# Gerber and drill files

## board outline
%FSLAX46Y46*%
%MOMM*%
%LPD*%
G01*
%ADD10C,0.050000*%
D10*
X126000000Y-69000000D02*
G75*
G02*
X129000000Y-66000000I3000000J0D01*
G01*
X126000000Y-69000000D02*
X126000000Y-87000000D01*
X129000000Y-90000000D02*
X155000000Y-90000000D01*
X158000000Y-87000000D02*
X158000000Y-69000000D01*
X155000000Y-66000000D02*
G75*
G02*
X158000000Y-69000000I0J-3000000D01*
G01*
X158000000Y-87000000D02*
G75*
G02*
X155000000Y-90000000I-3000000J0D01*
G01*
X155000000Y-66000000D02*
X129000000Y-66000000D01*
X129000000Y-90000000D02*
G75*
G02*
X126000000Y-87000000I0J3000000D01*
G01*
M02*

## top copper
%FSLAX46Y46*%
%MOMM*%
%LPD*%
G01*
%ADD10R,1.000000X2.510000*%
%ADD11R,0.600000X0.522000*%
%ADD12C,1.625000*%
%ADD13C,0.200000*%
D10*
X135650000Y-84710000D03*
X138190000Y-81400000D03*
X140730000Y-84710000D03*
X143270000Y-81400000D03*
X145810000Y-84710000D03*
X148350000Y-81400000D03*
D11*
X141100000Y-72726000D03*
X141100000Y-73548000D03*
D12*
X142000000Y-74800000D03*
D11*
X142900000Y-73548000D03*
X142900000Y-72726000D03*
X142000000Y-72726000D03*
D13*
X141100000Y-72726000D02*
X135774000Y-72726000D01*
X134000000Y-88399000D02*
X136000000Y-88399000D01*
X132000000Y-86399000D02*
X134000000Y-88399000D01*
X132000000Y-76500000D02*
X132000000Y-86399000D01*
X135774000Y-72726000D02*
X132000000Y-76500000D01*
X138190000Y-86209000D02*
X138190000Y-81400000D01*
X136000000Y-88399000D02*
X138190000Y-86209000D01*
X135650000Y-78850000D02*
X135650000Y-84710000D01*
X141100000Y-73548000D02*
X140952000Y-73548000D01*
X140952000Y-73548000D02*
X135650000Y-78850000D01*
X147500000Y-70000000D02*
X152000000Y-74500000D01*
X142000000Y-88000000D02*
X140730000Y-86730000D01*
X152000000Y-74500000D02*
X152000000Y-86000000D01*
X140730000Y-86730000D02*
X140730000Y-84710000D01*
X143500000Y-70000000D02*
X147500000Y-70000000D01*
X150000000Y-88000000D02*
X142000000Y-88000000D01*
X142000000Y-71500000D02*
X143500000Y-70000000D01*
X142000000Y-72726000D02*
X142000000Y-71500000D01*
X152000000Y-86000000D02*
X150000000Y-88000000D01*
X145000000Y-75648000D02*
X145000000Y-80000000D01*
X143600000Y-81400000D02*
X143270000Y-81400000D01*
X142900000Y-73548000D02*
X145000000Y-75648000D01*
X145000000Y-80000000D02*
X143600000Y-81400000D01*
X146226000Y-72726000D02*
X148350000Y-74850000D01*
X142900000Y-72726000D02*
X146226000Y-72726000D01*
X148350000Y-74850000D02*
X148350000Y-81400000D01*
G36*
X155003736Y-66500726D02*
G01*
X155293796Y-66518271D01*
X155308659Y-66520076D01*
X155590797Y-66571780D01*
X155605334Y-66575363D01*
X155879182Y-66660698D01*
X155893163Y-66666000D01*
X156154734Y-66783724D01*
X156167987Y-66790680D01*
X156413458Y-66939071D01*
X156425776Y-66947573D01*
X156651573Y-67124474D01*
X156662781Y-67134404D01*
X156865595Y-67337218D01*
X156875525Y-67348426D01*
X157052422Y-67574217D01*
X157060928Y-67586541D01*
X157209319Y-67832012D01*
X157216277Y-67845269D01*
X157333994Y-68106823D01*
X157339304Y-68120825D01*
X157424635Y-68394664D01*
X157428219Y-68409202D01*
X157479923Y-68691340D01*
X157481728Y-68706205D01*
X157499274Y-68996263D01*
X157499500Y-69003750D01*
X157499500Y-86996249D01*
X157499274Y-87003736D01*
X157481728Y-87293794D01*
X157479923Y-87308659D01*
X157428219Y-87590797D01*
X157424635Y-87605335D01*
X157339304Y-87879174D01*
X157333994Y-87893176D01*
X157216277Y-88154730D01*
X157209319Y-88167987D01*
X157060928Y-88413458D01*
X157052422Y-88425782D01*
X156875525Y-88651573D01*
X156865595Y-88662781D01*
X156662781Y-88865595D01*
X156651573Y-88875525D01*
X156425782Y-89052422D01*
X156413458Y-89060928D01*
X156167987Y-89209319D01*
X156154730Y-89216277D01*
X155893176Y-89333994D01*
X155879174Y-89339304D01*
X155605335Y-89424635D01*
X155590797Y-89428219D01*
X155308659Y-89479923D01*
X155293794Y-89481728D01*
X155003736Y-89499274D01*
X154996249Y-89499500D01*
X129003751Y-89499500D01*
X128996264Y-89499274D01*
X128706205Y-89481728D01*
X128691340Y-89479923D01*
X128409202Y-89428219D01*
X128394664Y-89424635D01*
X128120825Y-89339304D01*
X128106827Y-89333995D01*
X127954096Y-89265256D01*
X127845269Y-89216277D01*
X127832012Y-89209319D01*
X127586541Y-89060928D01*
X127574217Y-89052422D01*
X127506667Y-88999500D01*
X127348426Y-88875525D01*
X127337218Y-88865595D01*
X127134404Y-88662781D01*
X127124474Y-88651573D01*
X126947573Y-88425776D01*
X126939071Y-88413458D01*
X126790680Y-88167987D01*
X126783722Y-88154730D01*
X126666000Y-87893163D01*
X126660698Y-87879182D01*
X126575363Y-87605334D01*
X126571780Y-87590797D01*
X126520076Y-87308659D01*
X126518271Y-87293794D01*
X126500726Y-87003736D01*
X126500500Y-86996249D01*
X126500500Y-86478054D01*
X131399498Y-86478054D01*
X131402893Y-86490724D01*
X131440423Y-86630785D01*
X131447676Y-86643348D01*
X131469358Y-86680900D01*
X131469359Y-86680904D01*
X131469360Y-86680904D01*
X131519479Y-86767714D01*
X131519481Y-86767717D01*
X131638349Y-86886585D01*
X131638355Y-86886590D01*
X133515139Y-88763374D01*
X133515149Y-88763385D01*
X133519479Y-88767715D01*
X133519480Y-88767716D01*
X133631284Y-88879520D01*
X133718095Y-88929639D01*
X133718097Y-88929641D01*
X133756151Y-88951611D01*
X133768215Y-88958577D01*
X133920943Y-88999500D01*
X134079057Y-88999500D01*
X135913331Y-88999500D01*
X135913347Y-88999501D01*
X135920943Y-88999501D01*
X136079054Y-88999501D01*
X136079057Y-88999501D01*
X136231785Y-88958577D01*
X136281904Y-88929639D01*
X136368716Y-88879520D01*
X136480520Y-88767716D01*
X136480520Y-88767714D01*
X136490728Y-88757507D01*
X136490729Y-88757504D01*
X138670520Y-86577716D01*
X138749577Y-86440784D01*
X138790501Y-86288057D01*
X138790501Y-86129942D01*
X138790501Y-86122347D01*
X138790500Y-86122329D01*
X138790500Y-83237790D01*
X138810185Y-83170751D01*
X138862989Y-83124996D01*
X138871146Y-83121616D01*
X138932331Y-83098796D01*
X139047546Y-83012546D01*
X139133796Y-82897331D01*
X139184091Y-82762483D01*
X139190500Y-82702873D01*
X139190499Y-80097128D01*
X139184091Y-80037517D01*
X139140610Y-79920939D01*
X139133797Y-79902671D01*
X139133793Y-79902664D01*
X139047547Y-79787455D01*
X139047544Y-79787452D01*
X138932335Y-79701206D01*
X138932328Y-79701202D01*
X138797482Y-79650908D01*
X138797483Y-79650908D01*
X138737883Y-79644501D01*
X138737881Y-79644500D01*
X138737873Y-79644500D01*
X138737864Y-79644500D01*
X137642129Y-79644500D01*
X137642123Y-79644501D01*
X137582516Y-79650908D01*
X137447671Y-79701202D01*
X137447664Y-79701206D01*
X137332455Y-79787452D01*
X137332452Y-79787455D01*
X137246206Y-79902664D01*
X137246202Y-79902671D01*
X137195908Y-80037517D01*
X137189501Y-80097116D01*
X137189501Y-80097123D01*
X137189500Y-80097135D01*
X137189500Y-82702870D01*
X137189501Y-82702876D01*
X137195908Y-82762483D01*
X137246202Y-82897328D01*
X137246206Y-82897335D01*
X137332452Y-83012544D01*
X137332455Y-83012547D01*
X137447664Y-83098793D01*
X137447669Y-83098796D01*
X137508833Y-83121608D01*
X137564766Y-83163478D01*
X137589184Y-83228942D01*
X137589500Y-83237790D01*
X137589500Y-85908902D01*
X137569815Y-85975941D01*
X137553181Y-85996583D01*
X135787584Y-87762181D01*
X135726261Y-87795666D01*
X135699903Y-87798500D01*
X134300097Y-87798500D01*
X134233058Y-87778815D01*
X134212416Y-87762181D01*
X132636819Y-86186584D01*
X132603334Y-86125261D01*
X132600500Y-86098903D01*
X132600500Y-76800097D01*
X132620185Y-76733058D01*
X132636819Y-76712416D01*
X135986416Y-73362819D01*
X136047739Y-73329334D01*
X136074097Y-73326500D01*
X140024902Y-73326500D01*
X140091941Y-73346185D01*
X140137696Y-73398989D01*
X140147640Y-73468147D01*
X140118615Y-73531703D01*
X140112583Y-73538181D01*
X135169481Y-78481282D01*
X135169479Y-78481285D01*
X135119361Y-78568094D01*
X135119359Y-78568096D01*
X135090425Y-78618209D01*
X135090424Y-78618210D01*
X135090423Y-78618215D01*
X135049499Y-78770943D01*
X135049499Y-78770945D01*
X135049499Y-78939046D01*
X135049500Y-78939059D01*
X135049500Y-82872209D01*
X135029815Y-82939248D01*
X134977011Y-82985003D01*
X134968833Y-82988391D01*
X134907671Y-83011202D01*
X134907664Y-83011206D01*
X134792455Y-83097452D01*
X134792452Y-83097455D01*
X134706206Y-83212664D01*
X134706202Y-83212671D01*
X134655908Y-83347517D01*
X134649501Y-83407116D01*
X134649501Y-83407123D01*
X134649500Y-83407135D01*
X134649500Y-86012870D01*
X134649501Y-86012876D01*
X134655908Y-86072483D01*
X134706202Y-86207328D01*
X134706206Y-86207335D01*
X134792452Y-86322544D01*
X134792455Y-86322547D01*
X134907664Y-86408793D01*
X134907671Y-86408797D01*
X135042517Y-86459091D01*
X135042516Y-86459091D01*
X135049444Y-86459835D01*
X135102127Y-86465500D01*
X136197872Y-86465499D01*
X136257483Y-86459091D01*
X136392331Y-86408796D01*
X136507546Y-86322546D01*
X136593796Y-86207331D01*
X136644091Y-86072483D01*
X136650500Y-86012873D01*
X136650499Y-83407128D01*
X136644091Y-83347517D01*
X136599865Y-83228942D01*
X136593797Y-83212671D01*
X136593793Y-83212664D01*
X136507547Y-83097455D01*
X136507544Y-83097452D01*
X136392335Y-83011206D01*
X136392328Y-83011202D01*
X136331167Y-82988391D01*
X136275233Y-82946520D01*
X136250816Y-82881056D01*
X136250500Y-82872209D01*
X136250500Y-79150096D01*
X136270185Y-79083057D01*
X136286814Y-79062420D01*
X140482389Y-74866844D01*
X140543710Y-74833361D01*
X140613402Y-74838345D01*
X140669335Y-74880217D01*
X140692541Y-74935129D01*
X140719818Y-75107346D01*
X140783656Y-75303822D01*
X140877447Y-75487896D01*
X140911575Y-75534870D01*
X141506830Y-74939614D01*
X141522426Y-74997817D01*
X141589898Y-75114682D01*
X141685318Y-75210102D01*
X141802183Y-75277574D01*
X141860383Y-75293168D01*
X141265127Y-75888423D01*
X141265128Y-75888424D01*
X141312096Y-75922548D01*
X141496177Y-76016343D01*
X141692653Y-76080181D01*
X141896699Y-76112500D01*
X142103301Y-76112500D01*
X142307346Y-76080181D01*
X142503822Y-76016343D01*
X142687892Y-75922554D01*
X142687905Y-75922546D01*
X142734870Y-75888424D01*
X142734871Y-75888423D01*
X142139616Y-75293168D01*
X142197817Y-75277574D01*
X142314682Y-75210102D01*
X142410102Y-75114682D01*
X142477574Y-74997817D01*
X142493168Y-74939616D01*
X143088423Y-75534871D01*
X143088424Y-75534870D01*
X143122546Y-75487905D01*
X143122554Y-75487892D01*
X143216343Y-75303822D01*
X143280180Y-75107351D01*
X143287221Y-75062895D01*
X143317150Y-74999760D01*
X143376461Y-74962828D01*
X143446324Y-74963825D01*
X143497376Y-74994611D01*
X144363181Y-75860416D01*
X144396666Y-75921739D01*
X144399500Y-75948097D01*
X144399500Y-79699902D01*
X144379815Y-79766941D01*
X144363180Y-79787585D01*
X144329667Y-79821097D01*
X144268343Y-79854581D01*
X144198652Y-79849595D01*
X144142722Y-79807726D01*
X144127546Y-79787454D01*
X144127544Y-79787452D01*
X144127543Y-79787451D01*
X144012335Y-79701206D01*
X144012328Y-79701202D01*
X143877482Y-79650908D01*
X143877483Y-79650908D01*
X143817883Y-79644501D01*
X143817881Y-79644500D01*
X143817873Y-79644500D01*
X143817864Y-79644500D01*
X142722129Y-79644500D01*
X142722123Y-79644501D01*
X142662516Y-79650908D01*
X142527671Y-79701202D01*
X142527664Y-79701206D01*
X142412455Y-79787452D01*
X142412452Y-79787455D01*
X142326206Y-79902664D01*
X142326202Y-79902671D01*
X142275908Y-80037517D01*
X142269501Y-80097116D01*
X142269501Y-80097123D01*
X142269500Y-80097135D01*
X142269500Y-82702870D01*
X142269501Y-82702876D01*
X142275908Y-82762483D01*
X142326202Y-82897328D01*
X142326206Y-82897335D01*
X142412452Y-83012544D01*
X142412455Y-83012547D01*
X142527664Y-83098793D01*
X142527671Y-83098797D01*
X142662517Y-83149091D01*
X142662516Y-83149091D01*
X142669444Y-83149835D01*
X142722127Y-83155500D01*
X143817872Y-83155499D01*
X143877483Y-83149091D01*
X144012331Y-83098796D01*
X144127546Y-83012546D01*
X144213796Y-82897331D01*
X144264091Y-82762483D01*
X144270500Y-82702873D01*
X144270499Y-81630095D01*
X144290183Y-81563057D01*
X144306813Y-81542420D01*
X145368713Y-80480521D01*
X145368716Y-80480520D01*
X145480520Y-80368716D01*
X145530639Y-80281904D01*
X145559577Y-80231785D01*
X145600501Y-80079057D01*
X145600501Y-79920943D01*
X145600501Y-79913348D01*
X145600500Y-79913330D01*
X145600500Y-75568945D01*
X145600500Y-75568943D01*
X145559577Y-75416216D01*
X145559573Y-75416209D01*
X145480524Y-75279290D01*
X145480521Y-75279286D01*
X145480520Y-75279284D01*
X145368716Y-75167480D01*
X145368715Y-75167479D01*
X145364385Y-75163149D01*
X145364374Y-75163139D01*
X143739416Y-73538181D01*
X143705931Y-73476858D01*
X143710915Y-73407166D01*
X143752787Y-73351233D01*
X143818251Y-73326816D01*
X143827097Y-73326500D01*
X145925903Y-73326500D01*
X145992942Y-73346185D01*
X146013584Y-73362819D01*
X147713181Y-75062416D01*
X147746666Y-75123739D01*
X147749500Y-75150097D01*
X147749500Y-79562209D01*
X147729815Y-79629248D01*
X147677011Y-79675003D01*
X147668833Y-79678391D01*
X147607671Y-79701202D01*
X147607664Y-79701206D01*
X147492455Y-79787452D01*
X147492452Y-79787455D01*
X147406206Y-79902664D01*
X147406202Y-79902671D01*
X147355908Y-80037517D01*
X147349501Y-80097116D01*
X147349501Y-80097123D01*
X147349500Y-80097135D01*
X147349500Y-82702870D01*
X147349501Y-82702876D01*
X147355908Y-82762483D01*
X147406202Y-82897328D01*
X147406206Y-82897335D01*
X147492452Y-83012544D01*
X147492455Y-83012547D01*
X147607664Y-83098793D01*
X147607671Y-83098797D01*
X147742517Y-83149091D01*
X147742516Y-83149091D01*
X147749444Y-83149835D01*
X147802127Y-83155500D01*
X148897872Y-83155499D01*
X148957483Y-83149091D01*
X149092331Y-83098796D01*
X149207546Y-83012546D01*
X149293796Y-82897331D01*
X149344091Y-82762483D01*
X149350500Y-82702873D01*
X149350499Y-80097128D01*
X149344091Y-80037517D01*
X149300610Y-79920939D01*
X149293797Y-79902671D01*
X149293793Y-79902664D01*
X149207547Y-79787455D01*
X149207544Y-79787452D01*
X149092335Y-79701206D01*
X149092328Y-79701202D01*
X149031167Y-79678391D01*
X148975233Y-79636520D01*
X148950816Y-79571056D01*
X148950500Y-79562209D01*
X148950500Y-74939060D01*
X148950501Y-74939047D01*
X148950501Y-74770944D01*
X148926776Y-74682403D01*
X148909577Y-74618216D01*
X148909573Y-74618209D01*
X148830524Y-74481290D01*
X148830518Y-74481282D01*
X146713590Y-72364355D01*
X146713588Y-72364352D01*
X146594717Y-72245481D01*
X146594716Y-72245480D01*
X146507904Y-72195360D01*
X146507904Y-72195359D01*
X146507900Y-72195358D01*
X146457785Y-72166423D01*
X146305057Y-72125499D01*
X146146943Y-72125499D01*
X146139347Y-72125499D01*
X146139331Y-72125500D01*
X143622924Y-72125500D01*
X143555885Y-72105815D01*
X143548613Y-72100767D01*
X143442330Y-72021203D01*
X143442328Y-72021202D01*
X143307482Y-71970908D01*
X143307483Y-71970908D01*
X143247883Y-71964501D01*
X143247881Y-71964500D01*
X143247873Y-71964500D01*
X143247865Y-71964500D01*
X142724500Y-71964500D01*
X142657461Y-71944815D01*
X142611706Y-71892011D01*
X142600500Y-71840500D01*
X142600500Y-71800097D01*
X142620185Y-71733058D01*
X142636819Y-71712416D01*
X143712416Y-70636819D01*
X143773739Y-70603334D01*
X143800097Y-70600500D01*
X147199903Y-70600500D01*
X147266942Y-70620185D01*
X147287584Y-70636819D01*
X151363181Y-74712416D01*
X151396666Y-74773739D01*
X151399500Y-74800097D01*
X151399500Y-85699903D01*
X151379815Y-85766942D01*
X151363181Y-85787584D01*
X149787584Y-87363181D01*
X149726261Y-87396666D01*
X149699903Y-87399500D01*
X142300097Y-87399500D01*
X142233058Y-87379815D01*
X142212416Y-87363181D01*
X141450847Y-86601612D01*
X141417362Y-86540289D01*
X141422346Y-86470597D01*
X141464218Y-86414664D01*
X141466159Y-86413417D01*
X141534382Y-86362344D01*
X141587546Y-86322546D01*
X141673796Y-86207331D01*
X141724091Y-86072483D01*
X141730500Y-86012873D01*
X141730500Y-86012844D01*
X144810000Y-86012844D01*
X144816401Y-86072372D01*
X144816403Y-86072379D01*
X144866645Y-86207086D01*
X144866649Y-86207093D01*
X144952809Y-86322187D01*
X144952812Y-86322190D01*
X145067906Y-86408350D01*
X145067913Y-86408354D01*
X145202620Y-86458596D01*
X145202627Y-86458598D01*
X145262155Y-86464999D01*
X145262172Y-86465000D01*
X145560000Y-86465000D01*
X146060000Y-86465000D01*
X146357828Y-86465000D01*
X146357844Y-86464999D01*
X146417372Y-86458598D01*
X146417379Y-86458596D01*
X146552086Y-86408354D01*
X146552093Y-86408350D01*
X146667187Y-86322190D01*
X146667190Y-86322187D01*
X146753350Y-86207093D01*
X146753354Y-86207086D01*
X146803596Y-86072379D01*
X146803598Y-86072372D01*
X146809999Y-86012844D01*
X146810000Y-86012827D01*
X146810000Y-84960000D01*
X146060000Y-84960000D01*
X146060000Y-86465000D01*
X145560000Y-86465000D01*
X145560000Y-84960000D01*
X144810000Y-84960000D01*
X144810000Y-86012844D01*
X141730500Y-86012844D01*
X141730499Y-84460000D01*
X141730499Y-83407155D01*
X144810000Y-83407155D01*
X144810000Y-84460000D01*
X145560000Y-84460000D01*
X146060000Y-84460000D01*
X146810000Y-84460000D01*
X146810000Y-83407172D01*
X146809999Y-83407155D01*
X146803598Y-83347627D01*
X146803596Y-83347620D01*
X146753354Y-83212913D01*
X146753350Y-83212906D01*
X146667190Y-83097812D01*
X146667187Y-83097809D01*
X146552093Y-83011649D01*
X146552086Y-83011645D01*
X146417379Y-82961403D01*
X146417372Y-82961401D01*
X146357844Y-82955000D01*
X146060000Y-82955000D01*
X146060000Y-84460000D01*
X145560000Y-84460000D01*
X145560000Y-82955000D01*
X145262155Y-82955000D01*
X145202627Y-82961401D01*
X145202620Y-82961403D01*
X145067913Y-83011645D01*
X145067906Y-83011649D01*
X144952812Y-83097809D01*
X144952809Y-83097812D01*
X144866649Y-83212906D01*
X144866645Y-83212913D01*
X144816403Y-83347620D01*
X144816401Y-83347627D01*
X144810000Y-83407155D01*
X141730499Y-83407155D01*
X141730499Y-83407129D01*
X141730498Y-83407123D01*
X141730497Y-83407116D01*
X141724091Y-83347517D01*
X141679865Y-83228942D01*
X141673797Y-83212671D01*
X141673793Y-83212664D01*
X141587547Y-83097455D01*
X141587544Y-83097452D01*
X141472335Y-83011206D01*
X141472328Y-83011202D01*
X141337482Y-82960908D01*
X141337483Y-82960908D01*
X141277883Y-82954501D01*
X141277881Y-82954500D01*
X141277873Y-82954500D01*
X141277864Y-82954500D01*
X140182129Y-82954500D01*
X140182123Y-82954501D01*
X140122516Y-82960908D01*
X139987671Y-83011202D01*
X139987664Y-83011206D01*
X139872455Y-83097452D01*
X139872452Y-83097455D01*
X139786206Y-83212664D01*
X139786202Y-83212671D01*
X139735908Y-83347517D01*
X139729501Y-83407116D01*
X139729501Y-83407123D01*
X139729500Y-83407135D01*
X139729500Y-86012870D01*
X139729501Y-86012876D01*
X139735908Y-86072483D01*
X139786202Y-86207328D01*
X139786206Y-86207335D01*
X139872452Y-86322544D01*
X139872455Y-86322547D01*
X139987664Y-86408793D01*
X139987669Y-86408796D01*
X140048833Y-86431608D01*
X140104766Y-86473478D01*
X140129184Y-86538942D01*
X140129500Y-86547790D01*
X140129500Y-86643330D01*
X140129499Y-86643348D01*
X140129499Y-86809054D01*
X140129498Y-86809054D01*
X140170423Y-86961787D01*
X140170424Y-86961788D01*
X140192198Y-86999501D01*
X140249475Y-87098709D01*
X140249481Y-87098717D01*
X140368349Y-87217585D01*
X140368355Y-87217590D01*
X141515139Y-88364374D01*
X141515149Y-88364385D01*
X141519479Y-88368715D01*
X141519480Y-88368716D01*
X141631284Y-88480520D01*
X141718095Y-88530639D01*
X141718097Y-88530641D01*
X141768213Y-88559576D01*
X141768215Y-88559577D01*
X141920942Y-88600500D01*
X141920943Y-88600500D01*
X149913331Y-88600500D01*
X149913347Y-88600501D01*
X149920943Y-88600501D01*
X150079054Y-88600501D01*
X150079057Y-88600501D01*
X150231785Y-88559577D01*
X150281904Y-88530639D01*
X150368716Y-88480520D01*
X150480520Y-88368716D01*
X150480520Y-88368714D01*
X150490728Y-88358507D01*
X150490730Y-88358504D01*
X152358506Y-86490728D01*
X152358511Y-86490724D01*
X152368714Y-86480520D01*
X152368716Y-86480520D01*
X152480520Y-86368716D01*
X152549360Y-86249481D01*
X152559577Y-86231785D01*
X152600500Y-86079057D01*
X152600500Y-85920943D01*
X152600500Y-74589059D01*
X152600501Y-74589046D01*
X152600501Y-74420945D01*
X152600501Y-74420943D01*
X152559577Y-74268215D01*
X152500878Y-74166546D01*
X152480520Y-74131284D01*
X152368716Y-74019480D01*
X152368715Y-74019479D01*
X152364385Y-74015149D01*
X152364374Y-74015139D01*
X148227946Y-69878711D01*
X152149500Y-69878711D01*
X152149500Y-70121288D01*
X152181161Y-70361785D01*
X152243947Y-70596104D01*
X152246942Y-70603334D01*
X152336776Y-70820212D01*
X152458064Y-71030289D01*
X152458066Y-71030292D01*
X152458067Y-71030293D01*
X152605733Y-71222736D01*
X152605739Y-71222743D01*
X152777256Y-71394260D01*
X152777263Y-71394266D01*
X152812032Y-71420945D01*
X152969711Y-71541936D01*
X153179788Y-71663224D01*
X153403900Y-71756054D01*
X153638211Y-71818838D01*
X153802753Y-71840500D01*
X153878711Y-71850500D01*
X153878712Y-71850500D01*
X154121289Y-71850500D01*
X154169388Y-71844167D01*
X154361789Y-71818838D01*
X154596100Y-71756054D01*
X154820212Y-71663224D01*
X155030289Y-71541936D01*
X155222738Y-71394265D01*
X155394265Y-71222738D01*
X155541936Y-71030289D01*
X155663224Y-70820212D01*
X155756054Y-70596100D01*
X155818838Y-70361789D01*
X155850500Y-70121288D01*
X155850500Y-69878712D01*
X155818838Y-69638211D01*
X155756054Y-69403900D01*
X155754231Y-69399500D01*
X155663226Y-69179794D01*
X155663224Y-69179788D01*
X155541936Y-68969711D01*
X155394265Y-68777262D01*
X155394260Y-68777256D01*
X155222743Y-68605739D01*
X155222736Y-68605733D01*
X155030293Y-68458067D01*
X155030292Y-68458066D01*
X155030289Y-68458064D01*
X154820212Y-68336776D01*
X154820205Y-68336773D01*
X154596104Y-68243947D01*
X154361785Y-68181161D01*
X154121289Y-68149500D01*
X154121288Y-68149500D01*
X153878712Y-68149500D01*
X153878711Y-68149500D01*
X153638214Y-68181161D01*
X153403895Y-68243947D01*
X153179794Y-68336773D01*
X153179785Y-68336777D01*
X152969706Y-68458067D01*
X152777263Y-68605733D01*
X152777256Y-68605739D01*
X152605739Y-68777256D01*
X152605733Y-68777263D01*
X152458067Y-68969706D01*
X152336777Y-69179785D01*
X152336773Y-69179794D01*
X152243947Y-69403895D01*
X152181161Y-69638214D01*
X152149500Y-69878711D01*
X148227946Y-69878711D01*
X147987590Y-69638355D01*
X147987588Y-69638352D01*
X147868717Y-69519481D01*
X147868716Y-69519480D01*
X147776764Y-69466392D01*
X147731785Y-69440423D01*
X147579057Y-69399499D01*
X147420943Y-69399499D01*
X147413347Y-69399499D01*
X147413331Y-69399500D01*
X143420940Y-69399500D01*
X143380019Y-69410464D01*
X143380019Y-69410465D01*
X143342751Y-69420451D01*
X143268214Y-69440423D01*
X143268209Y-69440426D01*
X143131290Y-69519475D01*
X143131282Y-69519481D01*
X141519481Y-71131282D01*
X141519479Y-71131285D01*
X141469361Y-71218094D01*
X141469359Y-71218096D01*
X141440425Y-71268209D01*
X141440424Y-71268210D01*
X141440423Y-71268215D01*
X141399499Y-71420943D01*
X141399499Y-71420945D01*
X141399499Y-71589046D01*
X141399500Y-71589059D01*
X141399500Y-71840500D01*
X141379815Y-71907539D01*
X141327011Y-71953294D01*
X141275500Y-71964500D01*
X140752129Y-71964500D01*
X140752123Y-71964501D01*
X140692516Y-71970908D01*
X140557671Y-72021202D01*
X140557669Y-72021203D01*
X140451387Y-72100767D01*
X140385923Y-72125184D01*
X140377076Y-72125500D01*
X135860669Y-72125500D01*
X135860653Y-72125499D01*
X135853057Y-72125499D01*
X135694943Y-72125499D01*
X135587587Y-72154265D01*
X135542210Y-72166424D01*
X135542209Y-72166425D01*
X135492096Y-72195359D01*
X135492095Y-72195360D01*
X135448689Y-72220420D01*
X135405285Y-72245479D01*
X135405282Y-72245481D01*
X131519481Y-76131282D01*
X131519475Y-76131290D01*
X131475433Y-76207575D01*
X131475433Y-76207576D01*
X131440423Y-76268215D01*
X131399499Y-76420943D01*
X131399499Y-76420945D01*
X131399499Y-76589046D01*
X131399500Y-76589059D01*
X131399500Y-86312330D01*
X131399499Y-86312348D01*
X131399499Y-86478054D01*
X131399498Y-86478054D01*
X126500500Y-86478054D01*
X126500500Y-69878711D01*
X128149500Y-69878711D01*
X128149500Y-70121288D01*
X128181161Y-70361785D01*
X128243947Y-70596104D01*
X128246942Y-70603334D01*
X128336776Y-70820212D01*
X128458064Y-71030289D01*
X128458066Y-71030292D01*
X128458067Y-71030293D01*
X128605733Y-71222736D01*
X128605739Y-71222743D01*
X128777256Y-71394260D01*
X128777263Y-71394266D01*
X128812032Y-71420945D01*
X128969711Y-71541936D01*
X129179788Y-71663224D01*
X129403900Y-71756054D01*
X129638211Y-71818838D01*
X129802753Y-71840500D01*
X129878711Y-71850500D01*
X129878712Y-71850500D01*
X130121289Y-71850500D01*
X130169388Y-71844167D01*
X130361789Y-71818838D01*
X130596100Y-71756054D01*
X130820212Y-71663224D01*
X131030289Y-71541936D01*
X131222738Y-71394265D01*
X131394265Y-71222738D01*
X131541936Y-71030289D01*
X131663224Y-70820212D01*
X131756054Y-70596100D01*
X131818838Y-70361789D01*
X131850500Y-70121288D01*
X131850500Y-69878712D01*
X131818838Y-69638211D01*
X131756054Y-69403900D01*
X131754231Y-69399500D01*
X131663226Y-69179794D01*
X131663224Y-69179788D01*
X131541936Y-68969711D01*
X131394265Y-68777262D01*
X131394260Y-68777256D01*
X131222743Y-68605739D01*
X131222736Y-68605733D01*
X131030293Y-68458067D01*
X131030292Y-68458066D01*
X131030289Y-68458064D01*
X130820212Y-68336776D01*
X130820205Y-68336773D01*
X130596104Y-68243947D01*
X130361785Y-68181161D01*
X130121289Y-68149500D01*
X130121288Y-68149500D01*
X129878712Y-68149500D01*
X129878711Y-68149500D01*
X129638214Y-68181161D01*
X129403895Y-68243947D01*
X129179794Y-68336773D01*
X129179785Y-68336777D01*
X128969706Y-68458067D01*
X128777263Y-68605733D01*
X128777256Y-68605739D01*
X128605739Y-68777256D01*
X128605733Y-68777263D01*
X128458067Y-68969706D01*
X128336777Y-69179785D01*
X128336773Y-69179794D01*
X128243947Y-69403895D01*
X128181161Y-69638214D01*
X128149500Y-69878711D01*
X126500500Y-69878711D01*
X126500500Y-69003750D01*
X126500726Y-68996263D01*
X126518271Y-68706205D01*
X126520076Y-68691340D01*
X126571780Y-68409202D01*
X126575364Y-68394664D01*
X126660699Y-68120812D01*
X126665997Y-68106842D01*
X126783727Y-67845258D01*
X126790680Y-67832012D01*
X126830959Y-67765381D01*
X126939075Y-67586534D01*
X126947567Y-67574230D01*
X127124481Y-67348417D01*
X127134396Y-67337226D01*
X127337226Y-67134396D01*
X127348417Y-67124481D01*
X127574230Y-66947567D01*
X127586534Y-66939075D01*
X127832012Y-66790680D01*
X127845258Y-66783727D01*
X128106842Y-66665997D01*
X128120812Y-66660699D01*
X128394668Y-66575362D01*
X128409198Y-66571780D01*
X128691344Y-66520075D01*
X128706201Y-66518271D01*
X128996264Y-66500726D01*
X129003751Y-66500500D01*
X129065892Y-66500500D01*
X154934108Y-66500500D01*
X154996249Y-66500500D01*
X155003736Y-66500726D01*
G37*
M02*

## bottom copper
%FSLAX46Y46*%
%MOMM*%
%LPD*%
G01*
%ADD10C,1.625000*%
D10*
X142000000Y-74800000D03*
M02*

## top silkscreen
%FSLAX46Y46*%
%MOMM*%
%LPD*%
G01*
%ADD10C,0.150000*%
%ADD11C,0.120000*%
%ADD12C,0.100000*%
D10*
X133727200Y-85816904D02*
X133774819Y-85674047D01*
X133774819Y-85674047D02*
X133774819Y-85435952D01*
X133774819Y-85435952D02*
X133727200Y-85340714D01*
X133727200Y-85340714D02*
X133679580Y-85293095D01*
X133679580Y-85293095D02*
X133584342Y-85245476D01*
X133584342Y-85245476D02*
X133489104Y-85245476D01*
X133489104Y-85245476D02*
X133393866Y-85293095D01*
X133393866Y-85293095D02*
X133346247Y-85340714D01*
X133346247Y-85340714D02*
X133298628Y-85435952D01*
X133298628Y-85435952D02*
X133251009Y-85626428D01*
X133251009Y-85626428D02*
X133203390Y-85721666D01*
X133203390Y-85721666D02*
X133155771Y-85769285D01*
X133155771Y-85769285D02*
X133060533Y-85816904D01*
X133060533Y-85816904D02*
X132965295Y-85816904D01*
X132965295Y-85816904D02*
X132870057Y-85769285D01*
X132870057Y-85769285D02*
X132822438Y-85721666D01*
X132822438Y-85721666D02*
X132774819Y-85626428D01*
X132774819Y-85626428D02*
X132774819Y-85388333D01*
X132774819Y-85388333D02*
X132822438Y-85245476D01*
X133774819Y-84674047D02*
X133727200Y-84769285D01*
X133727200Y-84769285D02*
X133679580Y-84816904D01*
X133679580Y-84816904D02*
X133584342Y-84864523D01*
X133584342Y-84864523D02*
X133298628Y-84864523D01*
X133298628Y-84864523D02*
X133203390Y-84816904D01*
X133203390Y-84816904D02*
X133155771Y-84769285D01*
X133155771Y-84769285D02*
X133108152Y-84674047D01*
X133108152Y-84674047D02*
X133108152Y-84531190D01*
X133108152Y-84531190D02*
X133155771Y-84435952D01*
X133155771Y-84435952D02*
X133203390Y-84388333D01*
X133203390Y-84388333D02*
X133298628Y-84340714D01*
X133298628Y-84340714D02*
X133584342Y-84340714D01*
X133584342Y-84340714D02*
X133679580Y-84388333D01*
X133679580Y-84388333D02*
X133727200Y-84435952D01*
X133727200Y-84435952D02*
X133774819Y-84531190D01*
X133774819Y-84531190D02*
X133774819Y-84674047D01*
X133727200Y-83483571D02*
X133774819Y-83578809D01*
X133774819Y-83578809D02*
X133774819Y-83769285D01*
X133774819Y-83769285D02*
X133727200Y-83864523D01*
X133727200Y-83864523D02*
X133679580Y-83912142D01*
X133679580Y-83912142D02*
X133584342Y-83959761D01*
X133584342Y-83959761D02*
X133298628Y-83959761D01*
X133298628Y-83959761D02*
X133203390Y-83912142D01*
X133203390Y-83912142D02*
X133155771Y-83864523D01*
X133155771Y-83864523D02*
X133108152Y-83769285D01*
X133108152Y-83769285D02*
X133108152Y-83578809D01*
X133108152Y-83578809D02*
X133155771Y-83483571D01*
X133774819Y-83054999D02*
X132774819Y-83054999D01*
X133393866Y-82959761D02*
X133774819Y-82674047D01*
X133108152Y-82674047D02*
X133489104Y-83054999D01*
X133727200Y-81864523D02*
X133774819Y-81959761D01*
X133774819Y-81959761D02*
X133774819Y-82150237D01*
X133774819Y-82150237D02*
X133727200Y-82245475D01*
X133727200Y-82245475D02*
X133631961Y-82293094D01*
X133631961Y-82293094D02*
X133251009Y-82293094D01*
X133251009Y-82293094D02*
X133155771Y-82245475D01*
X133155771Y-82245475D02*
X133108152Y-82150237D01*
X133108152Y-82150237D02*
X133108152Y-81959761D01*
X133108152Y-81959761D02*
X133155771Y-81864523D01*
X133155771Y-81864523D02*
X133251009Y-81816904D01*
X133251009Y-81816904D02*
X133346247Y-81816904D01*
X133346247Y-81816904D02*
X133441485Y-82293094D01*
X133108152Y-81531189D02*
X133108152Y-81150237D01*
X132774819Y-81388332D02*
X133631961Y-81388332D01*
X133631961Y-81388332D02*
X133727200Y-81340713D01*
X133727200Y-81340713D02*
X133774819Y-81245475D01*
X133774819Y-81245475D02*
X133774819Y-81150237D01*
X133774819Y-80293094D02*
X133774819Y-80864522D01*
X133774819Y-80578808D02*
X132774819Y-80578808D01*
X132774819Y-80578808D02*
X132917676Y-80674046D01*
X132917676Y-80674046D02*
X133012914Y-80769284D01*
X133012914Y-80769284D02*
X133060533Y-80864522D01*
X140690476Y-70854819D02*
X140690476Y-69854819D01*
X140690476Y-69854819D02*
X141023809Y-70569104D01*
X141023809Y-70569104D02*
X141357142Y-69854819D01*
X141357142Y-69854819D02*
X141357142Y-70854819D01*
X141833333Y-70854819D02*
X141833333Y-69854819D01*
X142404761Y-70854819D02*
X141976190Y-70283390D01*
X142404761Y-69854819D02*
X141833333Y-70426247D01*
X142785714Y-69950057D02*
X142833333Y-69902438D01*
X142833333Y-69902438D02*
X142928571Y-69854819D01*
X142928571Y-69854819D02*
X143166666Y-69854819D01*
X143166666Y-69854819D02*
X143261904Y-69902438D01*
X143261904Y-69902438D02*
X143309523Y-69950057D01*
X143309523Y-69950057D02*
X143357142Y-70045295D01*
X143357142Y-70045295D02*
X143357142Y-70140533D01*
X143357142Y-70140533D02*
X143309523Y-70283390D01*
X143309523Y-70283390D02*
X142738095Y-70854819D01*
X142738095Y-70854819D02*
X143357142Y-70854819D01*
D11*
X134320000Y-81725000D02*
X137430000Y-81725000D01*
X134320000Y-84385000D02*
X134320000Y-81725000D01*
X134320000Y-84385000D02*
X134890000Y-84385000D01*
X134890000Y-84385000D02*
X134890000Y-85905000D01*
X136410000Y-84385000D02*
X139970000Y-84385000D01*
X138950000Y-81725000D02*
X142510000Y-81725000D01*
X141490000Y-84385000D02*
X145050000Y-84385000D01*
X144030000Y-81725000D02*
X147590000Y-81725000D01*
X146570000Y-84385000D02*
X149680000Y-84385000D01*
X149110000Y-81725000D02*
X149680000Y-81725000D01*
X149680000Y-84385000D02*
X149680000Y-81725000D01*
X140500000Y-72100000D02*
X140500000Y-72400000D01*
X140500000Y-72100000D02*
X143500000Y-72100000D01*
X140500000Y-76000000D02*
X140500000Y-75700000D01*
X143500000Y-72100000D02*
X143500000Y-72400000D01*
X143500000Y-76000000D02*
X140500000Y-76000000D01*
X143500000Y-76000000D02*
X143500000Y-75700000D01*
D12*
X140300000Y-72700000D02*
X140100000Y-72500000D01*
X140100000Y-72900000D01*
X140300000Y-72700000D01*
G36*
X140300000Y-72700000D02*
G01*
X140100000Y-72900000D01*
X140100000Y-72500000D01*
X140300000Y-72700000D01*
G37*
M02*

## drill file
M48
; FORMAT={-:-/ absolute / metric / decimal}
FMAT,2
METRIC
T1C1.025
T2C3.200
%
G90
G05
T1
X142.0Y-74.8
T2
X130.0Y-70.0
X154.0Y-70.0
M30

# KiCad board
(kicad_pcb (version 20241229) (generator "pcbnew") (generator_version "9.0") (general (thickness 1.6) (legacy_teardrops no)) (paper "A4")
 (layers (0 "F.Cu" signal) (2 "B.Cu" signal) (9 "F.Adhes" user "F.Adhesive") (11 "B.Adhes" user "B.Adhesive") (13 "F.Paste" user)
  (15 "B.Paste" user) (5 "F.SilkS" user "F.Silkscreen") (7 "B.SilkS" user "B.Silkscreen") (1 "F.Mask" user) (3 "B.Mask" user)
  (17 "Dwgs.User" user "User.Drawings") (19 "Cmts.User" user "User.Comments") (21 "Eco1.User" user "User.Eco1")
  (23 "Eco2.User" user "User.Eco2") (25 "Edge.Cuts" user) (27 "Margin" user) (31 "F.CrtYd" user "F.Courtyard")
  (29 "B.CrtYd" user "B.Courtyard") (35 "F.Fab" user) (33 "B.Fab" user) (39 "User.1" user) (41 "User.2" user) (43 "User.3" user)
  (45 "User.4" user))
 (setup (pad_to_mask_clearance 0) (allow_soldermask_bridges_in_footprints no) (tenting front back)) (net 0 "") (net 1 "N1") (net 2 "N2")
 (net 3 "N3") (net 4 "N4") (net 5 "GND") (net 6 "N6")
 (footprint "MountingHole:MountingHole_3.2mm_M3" (layer "F.Cu") (at 130 70)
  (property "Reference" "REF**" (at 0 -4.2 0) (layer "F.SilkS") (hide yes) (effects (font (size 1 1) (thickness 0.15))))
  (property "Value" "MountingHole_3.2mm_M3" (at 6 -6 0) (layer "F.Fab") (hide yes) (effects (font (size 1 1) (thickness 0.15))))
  (pad "" np_thru_hole circle (at 0 0) (size 3.2 3.2) (drill 3.2) (layers "*.Cu" "*.Mask")))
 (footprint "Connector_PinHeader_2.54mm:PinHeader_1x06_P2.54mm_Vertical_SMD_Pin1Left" (layer "F.Cu") (at 142 83.055 90)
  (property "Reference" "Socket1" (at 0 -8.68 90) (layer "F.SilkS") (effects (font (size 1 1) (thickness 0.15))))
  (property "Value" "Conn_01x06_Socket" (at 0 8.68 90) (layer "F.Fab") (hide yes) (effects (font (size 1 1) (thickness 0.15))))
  (fp_line (start 1.33 -7.68) (end 1.33 -4.57) (stroke (width 0.12) (type solid)) (layer "F.SilkS"))
  (fp_line (start -1.33 -7.68) (end 1.33 -7.68) (stroke (width 0.12) (type solid)) (layer "F.SilkS"))
  (fp_line (start -1.33 -7.68) (end -1.33 -7.11) (stroke (width 0.12) (type solid)) (layer "F.SilkS"))
  (fp_line (start -1.33 -7.11) (end -2.85 -7.11) (stroke (width 0.12) (type solid)) (layer "F.SilkS"))
  (fp_line (start -1.33 -5.59) (end -1.33 -2.03) (stroke (width 0.12) (type solid)) (layer "F.SilkS"))
  (fp_line (start 1.33 -3.05) (end 1.33 0.51) (stroke (width 0.12) (type solid)) (layer "F.SilkS"))
  (fp_line (start -1.33 -0.51) (end -1.33 3.05) (stroke (width 0.12) (type solid)) (layer "F.SilkS"))
  (fp_line (start 1.33 2.03) (end 1.33 5.59) (stroke (width 0.12) (type solid)) (layer "F.SilkS"))
  (fp_line (start -1.33 4.57) (end -1.33 7.68) (stroke (width 0.12) (type solid)) (layer "F.SilkS"))
  (fp_line (start 1.33 7.11) (end 1.33 7.68) (stroke (width 0.12) (type solid)) (layer "F.SilkS"))
  (fp_line (start -1.33 7.68) (end 1.33 7.68) (stroke (width 0.12) (type solid)) (layer "F.SilkS"))
  (pad "1" smd rect (at -1.655 -6.35 90) (size 2.51 1) (layers "F.Cu" "F.Mask" "F.Paste") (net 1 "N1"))
  (pad "2" smd rect (at 1.655 -3.81 90) (size 2.51 1) (layers "F.Cu" "F.Mask" "F.Paste") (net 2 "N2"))
  (pad "3" smd rect (at -1.655 -1.27 90) (size 2.51 1) (layers "F.Cu" "F.Mask" "F.Paste") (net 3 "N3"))
  (pad "4" smd rect (at 1.655 1.27 90) (size 2.51 1) (layers "F.Cu" "F.Mask" "F.Paste") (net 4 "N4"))
  (pad "5" smd rect (at -1.655 3.81 90) (size 2.51 1) (layers "F.Cu" "F.Mask" "F.Paste") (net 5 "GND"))
  (pad "6" smd rect (at 1.655 6.35 90) (size 2.51 1) (layers "F.Cu" "F.Mask" "F.Paste") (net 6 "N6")))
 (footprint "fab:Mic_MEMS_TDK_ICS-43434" (layer "F.Cu") (at 142 74)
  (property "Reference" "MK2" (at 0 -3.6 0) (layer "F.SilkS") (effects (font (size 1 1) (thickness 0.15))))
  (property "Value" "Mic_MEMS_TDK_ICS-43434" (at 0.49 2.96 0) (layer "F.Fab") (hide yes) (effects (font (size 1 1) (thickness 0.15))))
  (fp_line (start -1.5 -1.9) (end -1.5 -1.6) (stroke (width 0.12) (type solid)) (layer "F.SilkS"))
  (fp_line (start -1.5 -1.9) (end 1.5 -1.9) (stroke (width 0.12) (type solid)) (layer "F.SilkS"))
  (fp_line (start -1.5 2) (end -1.5 1.7) (stroke (width 0.12) (type solid)) (layer "F.SilkS"))
  (fp_line (start 1.5 -1.9) (end 1.5 -1.6) (stroke (width 0.12) (type solid)) (layer "F.SilkS"))
  (fp_line (start 1.5 2) (end -1.5 2) (stroke (width 0.12) (type solid)) (layer "F.SilkS"))
  (fp_line (start 1.5 2) (end 1.5 1.7) (stroke (width 0.12) (type solid)) (layer "F.SilkS"))
  (fp_poly (pts (xy -1.7 -1.3) (xy -1.9 -1.5) (xy -1.9 -1.1)) (stroke (width 0.1) (type solid)) (fill yes) (layer "F.SilkS"))
  (pad "1" smd rect (at -0.9 -1.274) (size 0.6 0.522) (layers "F.Cu" "F.Mask" "F.Paste") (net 2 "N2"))
  (pad "2" smd rect (at -0.9 -0.452) (size 0.6 0.522) (layers "F.Cu" "F.Mask" "F.Paste") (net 1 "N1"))
  (pad "3" thru_hole circle (at 0 0.8) (size 1.625 1.625) (drill 1.025) (layers "*.Cu" "*.Mask") (remove_unused_layers no) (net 5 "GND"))
  (pad "4" smd rect (at 0.9 -0.452) (size 0.6 0.522) (layers "F.Cu" "F.Mask" "F.Paste") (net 4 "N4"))
  (pad "5" smd rect (at 0.9 -1.274) (size 0.6 0.522) (layers "F.Cu" "F.Mask" "F.Paste") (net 6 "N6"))
  (pad "6" smd rect (at 0 -1.274) (size 0.6 0.522) (layers "F.Cu" "F.Mask" "F.Paste") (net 3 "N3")))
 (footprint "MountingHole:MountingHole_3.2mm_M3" (layer "F.Cu") (at 154 70)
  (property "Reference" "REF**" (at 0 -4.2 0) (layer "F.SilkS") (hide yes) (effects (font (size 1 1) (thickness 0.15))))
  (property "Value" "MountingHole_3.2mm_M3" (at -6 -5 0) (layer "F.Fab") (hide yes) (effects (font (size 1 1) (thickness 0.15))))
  (pad "" np_thru_hole circle (at 0 0) (size 3.2 3.2) (drill 3.2) (layers "*.Cu" "*.Mask")))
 (gr_arc (start 126 69) (mid 126.87868 66.87868) (end 129 66) (stroke (width 0.05) (type default)) (layer "Edge.Cuts"))
 (gr_line (start 126 69) (end 126 87) (stroke (width 0.05) (type default)) (layer "Edge.Cuts"))
 (gr_line (start 129 90) (end 155 90) (stroke (width 0.05) (type default)) (layer "Edge.Cuts"))
 (gr_line (start 158 87) (end 158 69) (stroke (width 0.05) (type default)) (layer "Edge.Cuts"))
 (gr_arc (start 155 66) (mid 157.12132 66.87868) (end 158 69) (stroke (width 0.05) (type default)) (layer "Edge.Cuts"))
 (gr_arc (start 158 87) (mid 157.12132 89.12132) (end 155 90) (stroke (width 0.05) (type default)) (layer "Edge.Cuts"))
 (gr_line (start 155 66) (end 129 66) (stroke (width 0.05) (type default)) (layer "Edge.Cuts"))
 (gr_arc (start 129 90) (mid 126.87868 89.12132) (end 126 87) (stroke (width 0.05) (type default)) (layer "Edge.Cuts"))
 (segment (start 141.1 72.726) (end 135.774 72.726) (width 0.2) (layer "F.Cu") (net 2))
 (segment (start 134 88.399) (end 136 88.399) (width 0.2) (layer "F.Cu") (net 2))
 (segment (start 132 86.399) (end 134 88.399) (width 0.2) (layer "F.Cu") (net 2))
 (segment (start 132 76.5) (end 132 86.399) (width 0.2) (layer "F.Cu") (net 2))
 (segment (start 135.774 72.726) (end 132 76.5) (width 0.2) (layer "F.Cu") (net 2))
 (segment (start 138.19 86.209) (end 138.19 81.4) (width 0.2) (layer "F.Cu") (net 2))
 (segment (start 136 88.399) (end 138.19 86.209) (width 0.2) (layer "F.Cu") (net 2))
 (segment (start 135.65 78.85) (end 135.65 84.71) (width 0.2) (layer "F.Cu") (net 1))
 (segment (start 141.1 73.548) (end 140.952 73.548) (width 0.2) (layer "F.Cu") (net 1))
 (segment (start 140.952 73.548) (end 135.65 78.85) (width 0.2) (layer "F.Cu") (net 1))
 (segment (start 147.5 70) (end 152 74.5) (width 0.2) (layer "F.Cu") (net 3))
 (segment (start 142 88) (end 140.73 86.73) (width 0.2) (layer "F.Cu") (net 3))
 (segment (start 152 74.5) (end 152 86) (width 0.2) (layer "F.Cu") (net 3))
 (segment (start 140.73 86.73) (end 140.73 84.71) (width 0.2) (layer "F.Cu") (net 3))
 (segment (start 143.5 70) (end 147.5 70) (width 0.2) (layer "F.Cu") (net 3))
 (segment (start 150 88) (end 142 88) (width 0.2) (layer "F.Cu") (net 3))
 (segment (start 142 71.5) (end 143.5 70) (width 0.2) (layer "F.Cu") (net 3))
 (segment (start 142 72.726) (end 142 71.5) (width 0.2) (layer "F.Cu") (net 3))
 (segment (start 152 86) (end 150 88) (width 0.2) (layer "F.Cu") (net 3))
 (segment (start 145 75.648) (end 145 80) (width 0.2) (layer "F.Cu") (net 4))
 (segment (start 143.6 81.4) (end 143.27 81.4) (width 0.2) (layer "F.Cu") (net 4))
 (segment (start 142.9 73.548) (end 145 75.648) (width 0.2) (layer "F.Cu") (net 4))
 (segment (start 145 80) (end 143.6 81.4) (width 0.2) (layer "F.Cu") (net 4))
 (segment (start 146.226 72.726) (end 148.35 74.85) (width 0.2) (layer "F.Cu") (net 6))
 (segment (start 142.9 72.726) (end 146.226 72.726) (width 0.2) (layer "F.Cu") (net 6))
 (segment (start 148.35 74.85) (end 148.35 81.4) (width 0.2) (layer "F.Cu") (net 6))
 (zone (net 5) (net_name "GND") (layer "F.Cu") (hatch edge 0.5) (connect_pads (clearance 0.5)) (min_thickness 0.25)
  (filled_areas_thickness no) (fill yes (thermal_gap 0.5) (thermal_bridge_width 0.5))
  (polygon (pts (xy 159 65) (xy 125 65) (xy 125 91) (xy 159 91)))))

